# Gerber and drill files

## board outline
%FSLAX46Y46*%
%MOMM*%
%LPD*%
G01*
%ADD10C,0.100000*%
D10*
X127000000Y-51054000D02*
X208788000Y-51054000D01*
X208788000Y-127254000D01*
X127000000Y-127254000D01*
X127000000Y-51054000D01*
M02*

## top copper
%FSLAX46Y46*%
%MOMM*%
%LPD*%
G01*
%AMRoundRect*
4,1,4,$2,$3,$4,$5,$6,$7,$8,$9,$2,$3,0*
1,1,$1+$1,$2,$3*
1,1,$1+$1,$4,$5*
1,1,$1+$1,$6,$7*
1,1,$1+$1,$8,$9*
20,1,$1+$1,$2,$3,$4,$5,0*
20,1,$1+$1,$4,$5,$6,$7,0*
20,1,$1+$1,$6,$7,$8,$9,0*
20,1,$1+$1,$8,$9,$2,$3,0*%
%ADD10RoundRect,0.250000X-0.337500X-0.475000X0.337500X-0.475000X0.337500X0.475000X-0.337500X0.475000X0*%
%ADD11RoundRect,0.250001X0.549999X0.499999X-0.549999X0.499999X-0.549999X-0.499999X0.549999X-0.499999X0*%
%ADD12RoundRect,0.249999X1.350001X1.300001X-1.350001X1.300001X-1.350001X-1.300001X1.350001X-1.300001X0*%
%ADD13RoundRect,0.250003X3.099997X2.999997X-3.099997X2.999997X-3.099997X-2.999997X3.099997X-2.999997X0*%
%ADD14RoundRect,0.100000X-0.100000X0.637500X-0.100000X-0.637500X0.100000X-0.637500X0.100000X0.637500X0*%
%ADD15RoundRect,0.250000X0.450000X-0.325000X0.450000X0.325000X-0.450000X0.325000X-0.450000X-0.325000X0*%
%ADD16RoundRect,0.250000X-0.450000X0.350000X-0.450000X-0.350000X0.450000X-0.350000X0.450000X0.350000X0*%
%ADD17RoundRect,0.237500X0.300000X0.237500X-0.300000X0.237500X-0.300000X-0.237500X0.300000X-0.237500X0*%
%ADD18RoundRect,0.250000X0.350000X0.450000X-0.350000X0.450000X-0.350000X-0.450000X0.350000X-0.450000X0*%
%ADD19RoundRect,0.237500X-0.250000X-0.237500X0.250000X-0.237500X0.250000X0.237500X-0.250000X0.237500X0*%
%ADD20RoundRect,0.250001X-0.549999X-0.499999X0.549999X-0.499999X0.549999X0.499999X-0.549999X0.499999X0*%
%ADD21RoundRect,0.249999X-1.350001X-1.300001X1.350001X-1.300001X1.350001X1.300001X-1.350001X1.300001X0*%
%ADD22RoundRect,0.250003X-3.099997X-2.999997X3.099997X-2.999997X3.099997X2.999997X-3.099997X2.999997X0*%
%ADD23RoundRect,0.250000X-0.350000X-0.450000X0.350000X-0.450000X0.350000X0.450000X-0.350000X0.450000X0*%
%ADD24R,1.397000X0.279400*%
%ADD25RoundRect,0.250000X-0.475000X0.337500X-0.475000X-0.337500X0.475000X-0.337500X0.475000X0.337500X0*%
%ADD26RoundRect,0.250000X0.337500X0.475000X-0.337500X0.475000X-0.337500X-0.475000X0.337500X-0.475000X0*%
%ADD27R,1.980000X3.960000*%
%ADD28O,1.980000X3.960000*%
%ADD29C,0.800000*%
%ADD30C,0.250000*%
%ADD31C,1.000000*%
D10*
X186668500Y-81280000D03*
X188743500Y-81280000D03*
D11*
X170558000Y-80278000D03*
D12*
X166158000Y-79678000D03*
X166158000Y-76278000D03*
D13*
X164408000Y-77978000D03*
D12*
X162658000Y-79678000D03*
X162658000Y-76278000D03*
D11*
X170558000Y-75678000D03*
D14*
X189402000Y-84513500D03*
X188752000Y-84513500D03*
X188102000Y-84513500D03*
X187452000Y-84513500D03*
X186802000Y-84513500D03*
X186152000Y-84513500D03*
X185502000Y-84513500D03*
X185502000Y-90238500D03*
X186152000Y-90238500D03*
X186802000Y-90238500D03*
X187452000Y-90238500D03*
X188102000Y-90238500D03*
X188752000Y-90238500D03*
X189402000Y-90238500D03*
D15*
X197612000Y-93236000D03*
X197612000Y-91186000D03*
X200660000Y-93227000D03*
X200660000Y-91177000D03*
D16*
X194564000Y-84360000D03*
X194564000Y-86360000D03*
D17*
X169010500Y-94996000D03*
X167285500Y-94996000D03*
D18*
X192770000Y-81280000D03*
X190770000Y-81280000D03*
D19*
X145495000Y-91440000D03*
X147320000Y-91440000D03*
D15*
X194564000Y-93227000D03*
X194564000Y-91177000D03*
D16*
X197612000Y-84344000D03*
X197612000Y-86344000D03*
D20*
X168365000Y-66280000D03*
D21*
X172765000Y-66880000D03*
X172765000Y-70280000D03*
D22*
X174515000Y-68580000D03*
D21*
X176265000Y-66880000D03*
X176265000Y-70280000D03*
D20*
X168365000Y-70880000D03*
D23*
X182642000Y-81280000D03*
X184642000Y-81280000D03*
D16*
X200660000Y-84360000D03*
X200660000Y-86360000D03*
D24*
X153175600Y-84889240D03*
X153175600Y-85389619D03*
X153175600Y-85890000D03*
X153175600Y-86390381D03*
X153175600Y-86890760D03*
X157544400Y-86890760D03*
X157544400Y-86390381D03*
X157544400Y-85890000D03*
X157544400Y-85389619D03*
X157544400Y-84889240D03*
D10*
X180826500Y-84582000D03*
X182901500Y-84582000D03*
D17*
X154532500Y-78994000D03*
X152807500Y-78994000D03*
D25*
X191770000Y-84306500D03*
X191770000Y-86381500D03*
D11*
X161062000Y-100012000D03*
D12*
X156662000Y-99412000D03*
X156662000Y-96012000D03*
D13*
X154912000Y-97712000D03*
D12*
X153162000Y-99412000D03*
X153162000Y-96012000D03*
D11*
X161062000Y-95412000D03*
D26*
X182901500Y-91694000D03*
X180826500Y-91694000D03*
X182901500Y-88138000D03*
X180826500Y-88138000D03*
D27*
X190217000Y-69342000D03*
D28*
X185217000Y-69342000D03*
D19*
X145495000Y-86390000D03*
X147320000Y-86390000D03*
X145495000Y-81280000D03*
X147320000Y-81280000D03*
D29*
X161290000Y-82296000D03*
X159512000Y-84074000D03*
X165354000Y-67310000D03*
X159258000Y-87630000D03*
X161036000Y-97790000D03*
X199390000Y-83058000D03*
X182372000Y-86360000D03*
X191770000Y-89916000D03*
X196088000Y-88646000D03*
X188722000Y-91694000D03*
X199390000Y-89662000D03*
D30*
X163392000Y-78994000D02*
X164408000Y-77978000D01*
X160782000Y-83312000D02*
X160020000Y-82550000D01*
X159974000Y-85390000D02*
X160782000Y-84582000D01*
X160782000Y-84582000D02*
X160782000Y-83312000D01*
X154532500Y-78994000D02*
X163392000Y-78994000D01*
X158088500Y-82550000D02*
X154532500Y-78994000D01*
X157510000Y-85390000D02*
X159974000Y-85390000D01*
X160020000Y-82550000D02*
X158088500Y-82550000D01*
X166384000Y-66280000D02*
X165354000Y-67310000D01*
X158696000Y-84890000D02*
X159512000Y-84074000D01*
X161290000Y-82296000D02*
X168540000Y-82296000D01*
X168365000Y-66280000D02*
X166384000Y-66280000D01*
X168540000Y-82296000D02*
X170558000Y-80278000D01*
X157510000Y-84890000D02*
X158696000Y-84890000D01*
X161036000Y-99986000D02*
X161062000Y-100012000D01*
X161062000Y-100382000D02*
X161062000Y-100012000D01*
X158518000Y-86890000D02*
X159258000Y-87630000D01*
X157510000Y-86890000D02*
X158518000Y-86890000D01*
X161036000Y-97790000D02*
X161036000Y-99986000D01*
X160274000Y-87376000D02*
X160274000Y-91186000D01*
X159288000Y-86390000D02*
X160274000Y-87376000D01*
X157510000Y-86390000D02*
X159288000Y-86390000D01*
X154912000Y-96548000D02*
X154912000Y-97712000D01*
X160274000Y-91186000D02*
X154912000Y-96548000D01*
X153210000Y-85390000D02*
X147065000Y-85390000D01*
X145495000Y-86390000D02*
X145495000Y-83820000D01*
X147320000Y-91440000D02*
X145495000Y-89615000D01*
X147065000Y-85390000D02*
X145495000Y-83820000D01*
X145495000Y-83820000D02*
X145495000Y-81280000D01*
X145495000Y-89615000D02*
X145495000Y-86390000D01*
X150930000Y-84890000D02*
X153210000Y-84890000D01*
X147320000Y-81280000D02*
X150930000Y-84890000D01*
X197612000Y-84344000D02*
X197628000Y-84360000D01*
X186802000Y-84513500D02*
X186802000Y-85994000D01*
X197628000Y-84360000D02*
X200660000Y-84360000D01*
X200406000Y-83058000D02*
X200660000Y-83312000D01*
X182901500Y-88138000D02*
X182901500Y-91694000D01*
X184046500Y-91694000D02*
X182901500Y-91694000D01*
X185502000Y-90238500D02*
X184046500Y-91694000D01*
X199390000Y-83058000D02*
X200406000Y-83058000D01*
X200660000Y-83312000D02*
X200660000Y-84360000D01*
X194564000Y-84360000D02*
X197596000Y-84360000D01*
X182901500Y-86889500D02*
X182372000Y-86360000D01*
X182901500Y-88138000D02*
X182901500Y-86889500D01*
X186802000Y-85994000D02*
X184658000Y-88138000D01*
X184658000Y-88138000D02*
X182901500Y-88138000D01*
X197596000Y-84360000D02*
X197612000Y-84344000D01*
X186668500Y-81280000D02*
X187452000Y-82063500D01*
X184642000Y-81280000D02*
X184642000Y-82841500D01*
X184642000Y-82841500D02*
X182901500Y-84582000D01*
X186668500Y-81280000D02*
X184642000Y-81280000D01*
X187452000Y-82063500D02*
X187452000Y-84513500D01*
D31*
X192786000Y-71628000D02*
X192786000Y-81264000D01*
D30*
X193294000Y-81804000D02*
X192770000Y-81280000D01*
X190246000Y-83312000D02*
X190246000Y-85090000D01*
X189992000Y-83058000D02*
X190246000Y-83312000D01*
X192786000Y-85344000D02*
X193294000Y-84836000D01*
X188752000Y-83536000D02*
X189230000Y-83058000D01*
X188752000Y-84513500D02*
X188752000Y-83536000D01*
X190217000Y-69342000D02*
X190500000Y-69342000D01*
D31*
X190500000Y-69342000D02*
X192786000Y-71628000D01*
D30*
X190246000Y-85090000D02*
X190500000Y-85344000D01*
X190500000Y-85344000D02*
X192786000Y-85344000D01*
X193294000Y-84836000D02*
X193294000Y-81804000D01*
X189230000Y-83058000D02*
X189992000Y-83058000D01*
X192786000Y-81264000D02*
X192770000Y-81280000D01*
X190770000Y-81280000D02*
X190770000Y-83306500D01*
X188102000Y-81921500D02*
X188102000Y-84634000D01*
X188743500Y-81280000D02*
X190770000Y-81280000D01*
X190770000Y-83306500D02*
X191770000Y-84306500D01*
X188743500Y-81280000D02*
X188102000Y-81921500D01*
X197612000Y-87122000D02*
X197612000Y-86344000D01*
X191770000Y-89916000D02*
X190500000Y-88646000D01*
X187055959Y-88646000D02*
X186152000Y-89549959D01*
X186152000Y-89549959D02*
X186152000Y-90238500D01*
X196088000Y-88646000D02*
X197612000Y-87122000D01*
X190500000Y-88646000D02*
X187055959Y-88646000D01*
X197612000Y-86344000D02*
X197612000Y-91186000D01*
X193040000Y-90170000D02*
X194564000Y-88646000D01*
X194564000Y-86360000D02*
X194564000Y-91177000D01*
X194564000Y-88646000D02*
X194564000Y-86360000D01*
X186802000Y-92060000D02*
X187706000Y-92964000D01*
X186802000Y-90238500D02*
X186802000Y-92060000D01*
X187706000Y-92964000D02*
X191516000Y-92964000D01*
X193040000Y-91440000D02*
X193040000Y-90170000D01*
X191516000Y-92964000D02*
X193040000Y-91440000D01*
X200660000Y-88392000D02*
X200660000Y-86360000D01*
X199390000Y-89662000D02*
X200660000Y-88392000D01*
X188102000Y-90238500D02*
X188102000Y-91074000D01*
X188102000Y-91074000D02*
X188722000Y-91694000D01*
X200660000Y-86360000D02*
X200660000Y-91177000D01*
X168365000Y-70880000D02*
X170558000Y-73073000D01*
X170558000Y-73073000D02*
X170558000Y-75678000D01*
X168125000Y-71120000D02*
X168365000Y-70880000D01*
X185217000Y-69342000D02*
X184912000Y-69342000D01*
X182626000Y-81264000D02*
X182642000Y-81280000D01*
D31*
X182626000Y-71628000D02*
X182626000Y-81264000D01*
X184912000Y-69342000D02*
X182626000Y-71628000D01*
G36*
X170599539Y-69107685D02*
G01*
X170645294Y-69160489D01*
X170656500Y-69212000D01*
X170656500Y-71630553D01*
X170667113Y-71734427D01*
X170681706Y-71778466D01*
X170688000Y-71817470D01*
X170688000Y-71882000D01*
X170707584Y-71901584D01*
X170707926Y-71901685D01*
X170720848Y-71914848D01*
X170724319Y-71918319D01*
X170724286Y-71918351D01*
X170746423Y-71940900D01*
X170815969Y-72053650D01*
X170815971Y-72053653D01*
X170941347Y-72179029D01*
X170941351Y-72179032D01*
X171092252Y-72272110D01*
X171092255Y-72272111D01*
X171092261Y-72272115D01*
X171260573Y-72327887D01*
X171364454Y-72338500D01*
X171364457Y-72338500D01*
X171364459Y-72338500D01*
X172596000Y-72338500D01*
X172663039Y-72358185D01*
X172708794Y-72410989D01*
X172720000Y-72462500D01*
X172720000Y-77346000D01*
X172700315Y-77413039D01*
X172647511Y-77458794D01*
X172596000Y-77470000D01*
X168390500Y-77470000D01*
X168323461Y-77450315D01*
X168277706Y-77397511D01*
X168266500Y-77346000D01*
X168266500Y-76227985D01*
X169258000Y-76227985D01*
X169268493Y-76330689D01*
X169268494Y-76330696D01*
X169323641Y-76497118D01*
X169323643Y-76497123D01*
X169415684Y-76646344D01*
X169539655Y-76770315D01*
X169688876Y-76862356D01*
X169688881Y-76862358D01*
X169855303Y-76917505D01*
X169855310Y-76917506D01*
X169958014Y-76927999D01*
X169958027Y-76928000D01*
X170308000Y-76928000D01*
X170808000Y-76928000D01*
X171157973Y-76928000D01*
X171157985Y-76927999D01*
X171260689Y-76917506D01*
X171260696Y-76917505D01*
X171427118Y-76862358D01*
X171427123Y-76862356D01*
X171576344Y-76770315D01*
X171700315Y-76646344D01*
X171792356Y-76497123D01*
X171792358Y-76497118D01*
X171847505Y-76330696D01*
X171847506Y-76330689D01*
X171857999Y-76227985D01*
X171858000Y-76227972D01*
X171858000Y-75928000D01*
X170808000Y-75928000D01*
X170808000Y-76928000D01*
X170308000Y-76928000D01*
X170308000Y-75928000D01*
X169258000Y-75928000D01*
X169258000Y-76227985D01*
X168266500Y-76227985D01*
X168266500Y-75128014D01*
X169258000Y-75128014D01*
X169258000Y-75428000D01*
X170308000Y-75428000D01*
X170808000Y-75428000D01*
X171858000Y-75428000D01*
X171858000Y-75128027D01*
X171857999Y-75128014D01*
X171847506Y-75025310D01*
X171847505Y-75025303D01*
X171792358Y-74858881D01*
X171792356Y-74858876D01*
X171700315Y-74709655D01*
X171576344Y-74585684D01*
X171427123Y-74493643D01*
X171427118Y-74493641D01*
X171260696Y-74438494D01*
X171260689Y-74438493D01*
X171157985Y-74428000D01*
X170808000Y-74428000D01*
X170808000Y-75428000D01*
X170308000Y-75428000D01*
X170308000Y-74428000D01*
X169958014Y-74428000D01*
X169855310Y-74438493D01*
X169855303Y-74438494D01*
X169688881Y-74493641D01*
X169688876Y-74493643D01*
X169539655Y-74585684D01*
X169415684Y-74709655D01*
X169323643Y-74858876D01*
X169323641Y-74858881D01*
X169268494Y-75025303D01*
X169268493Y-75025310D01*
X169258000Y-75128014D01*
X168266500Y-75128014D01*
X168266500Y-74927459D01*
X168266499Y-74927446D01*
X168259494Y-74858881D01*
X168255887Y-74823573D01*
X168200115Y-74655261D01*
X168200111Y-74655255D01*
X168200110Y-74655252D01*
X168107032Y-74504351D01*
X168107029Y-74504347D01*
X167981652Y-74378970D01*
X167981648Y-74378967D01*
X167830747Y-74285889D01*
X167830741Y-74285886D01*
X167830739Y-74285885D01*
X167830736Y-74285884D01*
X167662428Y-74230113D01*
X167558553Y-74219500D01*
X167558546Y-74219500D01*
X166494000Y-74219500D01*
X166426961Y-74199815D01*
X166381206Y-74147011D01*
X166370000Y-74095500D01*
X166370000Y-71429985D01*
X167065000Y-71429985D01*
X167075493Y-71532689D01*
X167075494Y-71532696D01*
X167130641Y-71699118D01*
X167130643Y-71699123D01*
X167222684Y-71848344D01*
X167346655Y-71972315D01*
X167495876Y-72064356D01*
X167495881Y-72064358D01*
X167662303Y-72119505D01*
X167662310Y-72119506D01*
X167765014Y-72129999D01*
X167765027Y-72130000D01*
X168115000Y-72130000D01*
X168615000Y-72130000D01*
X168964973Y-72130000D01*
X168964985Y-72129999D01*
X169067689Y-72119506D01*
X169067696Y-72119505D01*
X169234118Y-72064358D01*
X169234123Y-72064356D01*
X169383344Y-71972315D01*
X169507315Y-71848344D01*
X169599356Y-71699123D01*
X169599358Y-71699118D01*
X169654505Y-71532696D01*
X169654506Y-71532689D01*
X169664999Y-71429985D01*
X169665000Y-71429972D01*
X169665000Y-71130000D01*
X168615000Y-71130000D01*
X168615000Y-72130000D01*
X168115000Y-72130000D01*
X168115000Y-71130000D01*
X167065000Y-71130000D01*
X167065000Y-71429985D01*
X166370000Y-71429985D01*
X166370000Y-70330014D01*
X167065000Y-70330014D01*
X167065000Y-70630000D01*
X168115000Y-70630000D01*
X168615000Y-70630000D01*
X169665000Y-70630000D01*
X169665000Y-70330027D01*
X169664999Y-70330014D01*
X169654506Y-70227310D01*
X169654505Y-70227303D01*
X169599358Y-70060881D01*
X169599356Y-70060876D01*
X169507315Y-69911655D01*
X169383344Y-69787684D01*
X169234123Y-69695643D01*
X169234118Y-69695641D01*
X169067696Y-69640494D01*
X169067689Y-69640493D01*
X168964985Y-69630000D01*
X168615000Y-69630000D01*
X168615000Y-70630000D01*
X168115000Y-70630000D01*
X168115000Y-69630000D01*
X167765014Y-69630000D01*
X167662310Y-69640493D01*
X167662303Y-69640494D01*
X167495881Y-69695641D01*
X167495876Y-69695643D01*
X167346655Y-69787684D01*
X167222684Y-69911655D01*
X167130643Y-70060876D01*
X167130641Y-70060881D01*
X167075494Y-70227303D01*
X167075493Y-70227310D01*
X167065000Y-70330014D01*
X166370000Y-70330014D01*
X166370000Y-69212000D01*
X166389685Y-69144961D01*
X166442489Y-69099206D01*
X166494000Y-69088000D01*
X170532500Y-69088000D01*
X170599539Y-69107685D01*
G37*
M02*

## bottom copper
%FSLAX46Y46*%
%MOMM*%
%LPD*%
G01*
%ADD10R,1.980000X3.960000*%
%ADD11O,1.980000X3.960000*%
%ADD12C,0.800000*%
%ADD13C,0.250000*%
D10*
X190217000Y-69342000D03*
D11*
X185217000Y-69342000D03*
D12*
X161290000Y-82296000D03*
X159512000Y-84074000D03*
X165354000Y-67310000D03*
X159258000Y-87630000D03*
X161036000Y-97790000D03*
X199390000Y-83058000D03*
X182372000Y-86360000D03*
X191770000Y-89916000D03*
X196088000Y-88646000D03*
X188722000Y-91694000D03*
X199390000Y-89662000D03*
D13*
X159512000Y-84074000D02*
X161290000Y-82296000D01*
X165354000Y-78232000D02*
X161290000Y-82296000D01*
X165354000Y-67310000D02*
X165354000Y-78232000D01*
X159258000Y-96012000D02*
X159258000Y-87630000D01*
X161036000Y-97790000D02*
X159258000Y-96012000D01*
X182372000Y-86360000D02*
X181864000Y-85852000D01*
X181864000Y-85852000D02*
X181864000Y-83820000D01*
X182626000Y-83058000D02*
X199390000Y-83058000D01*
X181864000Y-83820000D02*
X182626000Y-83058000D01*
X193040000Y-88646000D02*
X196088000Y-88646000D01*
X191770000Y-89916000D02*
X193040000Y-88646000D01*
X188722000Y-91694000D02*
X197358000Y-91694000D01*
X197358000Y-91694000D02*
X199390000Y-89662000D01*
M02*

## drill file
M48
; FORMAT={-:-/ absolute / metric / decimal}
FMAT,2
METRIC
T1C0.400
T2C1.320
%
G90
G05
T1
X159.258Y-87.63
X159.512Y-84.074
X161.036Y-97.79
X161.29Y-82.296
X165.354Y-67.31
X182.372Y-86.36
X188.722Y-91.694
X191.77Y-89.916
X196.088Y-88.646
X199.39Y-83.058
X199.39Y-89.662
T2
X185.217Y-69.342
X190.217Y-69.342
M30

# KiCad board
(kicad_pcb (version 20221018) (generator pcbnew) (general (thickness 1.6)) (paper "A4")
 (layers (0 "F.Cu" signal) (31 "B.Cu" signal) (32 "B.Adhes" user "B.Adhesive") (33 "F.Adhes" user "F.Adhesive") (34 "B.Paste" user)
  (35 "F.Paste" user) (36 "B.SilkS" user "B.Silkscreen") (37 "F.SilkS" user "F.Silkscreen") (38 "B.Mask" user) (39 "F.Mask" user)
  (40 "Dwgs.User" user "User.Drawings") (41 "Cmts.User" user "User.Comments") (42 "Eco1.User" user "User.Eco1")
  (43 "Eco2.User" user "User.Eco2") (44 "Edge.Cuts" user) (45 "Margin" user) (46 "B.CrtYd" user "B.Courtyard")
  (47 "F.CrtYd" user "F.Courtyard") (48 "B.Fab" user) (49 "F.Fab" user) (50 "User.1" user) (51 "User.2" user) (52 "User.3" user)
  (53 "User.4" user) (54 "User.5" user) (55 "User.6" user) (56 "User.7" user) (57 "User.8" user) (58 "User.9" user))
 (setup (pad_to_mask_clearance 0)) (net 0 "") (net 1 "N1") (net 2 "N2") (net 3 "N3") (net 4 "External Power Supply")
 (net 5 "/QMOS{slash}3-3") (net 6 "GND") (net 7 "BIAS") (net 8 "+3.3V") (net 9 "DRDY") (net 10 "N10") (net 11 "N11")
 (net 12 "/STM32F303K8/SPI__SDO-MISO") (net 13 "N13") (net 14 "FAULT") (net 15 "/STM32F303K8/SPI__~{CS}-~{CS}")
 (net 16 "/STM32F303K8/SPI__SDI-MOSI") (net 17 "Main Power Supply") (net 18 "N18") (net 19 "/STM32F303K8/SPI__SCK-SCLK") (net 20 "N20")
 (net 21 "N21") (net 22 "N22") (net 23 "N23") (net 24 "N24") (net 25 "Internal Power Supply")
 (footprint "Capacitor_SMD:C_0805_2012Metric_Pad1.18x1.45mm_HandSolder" (layer "F.Cu") (at 187.706 81.28)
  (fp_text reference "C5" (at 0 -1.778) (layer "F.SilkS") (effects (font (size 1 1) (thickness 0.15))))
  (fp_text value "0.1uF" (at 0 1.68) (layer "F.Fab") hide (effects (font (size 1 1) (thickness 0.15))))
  (pad "1" smd roundrect (at -1.0375 0) (size 1.175 1.45) (layers "F.Cu" "F.Paste" "F.Mask") (roundrect_rratio 0.212766) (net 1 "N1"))
  (pad "2" smd roundrect (at 1.0375 0) (size 1.175 1.45) (layers "F.Cu" "F.Paste" "F.Mask") (roundrect_rratio 0.212766) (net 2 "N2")))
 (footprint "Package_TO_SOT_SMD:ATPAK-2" (layer "F.Cu") (at 165.608 77.978 180)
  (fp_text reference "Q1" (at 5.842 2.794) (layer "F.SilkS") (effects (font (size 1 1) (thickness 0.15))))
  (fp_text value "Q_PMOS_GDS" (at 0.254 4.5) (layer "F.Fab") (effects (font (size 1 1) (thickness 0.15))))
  (pad "1" smd roundrect (at -4.95 -2.3 180) (size 1.6 1.5) (layers "F.Cu" "F.Paste" "F.Mask") (roundrect_rratio 0.166667) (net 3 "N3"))
  (pad "2" smd roundrect (at -0.55 -1.7 180) (size 3.2 3.1) (layers "F.Cu" "F.Paste") (roundrect_rratio 0.080645)
   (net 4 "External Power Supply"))
  (pad "2" smd roundrect (at -0.55 1.7 180) (size 3.2 3.1) (layers "F.Cu" "F.Paste") (roundrect_rratio 0.080645)
   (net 4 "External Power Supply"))
  (pad "2" smd roundrect (at 1.2 0 180) (size 6.7 6.5) (layers "F.Cu" "F.Mask") (roundrect_rratio 0.038462) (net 4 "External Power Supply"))
  (pad "2" smd roundrect (at 2.95 -1.7 180) (size 3.2 3.1) (layers "F.Cu" "F.Paste") (roundrect_rratio 0.080645)
   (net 4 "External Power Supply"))
  (pad "2" smd roundrect (at 2.95 1.7 180) (size 3.2 3.1) (layers "F.Cu" "F.Paste") (roundrect_rratio 0.080645)
   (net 4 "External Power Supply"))
  (pad "3" smd roundrect (at -4.95 2.3 180) (size 1.6 1.5) (layers "F.Cu" "F.Paste" "F.Mask") (roundrect_rratio 0.166667)
   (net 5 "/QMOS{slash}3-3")))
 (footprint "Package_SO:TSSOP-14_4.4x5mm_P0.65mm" (layer "F.Cu") (at 187.452 87.376 -90)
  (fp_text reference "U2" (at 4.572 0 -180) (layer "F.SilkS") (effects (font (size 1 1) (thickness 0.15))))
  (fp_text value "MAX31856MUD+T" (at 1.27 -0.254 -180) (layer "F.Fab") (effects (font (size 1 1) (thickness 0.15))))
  (pad "1" smd roundrect (at -2.8625 -1.95 270) (size 1.475 0.4) (layers "F.Cu" "F.Paste" "F.Mask") (roundrect_rratio 0.25) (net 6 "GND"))
  (pad "2" smd roundrect (at -2.8625 -1.3 270) (size 1.475 0.4) (layers "F.Cu" "F.Paste" "F.Mask") (roundrect_rratio 0.25) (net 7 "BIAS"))
  (pad "3" smd roundrect (at -2.8625 -0.65 270) (size 1.475 0.4) (layers "F.Cu" "F.Paste" "F.Mask") (roundrect_rratio 0.25) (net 2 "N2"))
  (pad "4" smd roundrect (at -2.8625 0 270) (size 1.475 0.4) (layers "F.Cu" "F.Paste" "F.Mask") (roundrect_rratio 0.25) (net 1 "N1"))
  (pad "5" smd roundrect (at -2.8625 0.65 270) (size 1.475 0.4) (layers "F.Cu" "F.Paste" "F.Mask") (roundrect_rratio 0.25) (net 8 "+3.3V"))
  (pad "6" smd roundrect (at -2.8625 1.3 270) (size 1.475 0.4) (layers "F.Cu" "F.Paste" "F.Mask") (roundrect_rratio 0.25))
  (pad "7" smd roundrect (at -2.8625 1.95 270) (size 1.475 0.4) (layers "F.Cu" "F.Paste" "F.Mask") (roundrect_rratio 0.25) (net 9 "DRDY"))
  (pad "8" smd roundrect (at 2.8625 1.95 270) (size 1.475 0.4) (layers "F.Cu" "F.Paste" "F.Mask") (roundrect_rratio 0.25) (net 8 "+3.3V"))
  (pad "9" smd roundrect (at 2.8625 1.3 270) (size 1.475 0.4) (layers "F.Cu" "F.Paste" "F.Mask") (roundrect_rratio 0.25) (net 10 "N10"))
  (pad "10" smd roundrect (at 2.8625 0.65 270) (size 1.475 0.4) (layers "F.Cu" "F.Paste" "F.Mask") (roundrect_rratio 0.25) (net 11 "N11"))
  (pad "11" smd roundrect (at 2.8625 0 270) (size 1.475 0.4) (layers "F.Cu" "F.Paste" "F.Mask") (roundrect_rratio 0.25)
   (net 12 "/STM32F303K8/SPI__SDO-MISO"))
  (pad "12" smd roundrect (at 2.8625 -0.65 270) (size 1.475 0.4) (layers "F.Cu" "F.Paste" "F.Mask") (roundrect_rratio 0.25) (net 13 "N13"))
  (pad "13" smd roundrect (at 2.8625 -1.3 270) (size 1.475 0.4) (layers "F.Cu" "F.Paste" "F.Mask") (roundrect_rratio 0.25) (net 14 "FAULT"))
  (pad "14" smd roundrect (at 2.8625 -1.95 270) (size 1.475 0.4) (layers "F.Cu" "F.Paste" "F.Mask") (roundrect_rratio 0.25) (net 6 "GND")))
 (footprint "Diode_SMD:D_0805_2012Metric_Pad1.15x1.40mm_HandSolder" (layer "F.Cu") (at 197.612 92.211 90)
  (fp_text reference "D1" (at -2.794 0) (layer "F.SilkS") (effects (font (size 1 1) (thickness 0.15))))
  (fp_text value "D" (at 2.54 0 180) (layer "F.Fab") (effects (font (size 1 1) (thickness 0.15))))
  (pad "1" smd roundrect (at -1.025 0 90) (size 1.15 1.4) (layers "F.Cu" "F.Paste" "F.Mask") (roundrect_rratio 0.217391)
   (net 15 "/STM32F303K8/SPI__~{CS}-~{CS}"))
  (pad "2" smd roundrect (at 1.025 0 90) (size 1.15 1.4) (layers "F.Cu" "F.Paste" "F.Mask") (roundrect_rratio 0.217391) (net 10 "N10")))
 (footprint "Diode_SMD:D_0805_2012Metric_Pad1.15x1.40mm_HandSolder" (layer "F.Cu") (at 200.66 92.202 90)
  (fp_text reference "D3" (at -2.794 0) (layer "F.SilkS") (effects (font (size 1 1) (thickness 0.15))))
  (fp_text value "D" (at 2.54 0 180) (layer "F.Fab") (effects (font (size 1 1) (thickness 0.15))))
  (pad "1" smd roundrect (at -1.025 0 90) (size 1.15 1.4) (layers "F.Cu" "F.Paste" "F.Mask") (roundrect_rratio 0.217391)
   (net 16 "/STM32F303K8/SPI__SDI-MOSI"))
  (pad "2" smd roundrect (at 1.025 0 90) (size 1.15 1.4) (layers "F.Cu" "F.Paste" "F.Mask") (roundrect_rratio 0.217391) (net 13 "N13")))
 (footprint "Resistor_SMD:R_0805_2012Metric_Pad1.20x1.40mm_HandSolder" (layer "F.Cu") (at 194.564 85.36 -90)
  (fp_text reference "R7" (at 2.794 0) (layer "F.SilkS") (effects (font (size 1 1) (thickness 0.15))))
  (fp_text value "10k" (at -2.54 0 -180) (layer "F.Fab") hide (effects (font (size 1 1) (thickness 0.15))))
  (pad "1" smd roundrect (at -1 0 270) (size 1.2 1.4) (layers "F.Cu" "F.Paste" "F.Mask") (roundrect_rratio 0.208333) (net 8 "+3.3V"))
  (pad "2" smd roundrect (at 1 0 270) (size 1.2 1.4) (layers "F.Cu" "F.Paste" "F.Mask") (roundrect_rratio 0.208333) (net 11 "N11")))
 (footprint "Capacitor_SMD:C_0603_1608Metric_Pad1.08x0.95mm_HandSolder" (layer "F.Cu") (at 168.148 94.996 180)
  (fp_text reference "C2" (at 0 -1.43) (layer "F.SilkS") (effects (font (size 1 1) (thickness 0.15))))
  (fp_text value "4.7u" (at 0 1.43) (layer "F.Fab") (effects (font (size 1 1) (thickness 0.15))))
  (pad "1" smd roundrect (at -0.8625 0 180) (size 1.075 0.95) (layers "F.Cu" "F.Paste" "F.Mask") (roundrect_rratio 0.25)
   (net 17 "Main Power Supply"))
  (pad "2" smd roundrect (at 0.8625 0 180) (size 1.075 0.95) (layers "F.Cu" "F.Paste" "F.Mask") (roundrect_rratio 0.25) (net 6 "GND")))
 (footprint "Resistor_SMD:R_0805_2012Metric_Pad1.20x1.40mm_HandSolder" (layer "F.Cu") (at 191.77 81.28 180)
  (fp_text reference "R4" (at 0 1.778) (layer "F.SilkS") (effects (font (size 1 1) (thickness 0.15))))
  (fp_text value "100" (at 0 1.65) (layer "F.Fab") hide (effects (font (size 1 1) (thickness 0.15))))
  (pad "1" smd roundrect (at -1 0 180) (size 1.2 1.4) (layers "F.Cu" "F.Paste" "F.Mask") (roundrect_rratio 0.208333) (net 7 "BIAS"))
  (pad "2" smd roundrect (at 1 0 180) (size 1.2 1.4) (layers "F.Cu" "F.Paste" "F.Mask") (roundrect_rratio 0.208333) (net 2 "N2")))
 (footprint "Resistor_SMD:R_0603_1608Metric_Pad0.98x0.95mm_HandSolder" (layer "F.Cu") (at 146.4075 91.44)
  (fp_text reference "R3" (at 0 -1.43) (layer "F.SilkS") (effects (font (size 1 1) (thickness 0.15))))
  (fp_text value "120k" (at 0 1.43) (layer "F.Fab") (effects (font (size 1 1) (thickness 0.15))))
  (pad "1" smd roundrect (at -0.9125 0) (size 0.975 0.95) (layers "F.Cu" "F.Paste" "F.Mask") (roundrect_rratio 0.25)
   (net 4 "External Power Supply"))
  (pad "2" smd roundrect (at 0.9125 0) (size 0.975 0.95) (layers "F.Cu" "F.Paste" "F.Mask") (roundrect_rratio 0.25) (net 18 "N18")))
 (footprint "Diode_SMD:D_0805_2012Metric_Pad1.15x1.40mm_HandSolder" (layer "F.Cu") (at 194.564 92.202 90)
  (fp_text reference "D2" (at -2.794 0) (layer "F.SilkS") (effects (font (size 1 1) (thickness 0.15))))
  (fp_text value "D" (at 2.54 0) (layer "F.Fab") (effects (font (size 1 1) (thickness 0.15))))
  (pad "1" smd roundrect (at -1.025 0 90) (size 1.15 1.4) (layers "F.Cu" "F.Paste" "F.Mask") (roundrect_rratio 0.217391)
   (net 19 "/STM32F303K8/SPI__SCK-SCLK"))
  (pad "2" smd roundrect (at 1.025 0 90) (size 1.15 1.4) (layers "F.Cu" "F.Paste" "F.Mask") (roundrect_rratio 0.217391) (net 11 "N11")))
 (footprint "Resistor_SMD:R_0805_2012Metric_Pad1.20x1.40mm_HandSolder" (layer "F.Cu") (at 197.612 85.344 -90)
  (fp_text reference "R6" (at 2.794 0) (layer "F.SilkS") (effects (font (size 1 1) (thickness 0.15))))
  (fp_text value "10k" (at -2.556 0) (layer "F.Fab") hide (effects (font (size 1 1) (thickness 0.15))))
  (pad "1" smd roundrect (at -1 0 270) (size 1.2 1.4) (layers "F.Cu" "F.Paste" "F.Mask") (roundrect_rratio 0.208333) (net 8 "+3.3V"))
  (pad "2" smd roundrect (at 1 0 270) (size 1.2 1.4) (layers "F.Cu" "F.Paste" "F.Mask") (roundrect_rratio 0.208333) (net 10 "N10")))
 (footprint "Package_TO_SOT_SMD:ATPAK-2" (layer "F.Cu") (at 173.315 68.58)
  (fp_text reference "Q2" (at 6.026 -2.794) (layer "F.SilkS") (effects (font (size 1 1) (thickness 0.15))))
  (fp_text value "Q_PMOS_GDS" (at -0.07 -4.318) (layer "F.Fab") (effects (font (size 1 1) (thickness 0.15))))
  (pad "1" smd roundrect (at -4.95 -2.3) (size 1.6 1.5) (layers "F.Cu" "F.Paste" "F.Mask") (roundrect_rratio 0.166667) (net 3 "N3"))
  (pad "2" smd roundrect (at -0.55 -1.7) (size 3.2 3.1) (layers "F.Cu" "F.Paste") (roundrect_rratio 0.080645) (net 17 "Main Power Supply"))
  (pad "2" smd roundrect (at -0.55 1.7) (size 3.2 3.1) (layers "F.Cu" "F.Paste") (roundrect_rratio 0.080645) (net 17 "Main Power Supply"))
  (pad "2" smd roundrect (at 1.2 0) (size 6.7 6.5) (layers "F.Cu" "F.Mask") (roundrect_rratio 0.038462) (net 17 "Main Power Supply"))
  (pad "2" smd roundrect (at 2.95 -1.7) (size 3.2 3.1) (layers "F.Cu" "F.Paste") (roundrect_rratio 0.080645) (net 17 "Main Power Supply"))
  (pad "2" smd roundrect (at 2.95 1.7) (size 3.2 3.1) (layers "F.Cu" "F.Paste") (roundrect_rratio 0.080645) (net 17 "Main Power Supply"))
  (pad "3" smd roundrect (at -4.95 2.3) (size 1.6 1.5) (layers "F.Cu" "F.Paste" "F.Mask") (roundrect_rratio 0.166667)
   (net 5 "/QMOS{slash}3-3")))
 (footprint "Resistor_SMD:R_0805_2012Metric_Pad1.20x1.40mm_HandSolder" (layer "F.Cu") (at 183.642 81.28)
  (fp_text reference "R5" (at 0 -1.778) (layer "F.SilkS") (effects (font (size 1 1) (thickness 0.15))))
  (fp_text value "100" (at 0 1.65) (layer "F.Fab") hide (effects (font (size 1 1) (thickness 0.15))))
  (pad "1" smd roundrect (at -1 0) (size 1.2 1.4) (layers "F.Cu" "F.Paste" "F.Mask") (roundrect_rratio 0.208333) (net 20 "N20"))
  (pad "2" smd roundrect (at 1 0) (size 1.2 1.4) (layers "F.Cu" "F.Paste" "F.Mask") (roundrect_rratio 0.208333) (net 1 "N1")))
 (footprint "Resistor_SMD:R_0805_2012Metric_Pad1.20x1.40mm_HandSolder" (layer "F.Cu") (at 200.66 85.36 -90)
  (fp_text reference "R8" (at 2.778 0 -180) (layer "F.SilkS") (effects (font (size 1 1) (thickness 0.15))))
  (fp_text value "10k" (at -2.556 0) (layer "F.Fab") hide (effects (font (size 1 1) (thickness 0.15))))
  (pad "1" smd roundrect (at -1 0 270) (size 1.2 1.4) (layers "F.Cu" "F.Paste" "F.Mask") (roundrect_rratio 0.208333) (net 8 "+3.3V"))
  (pad "2" smd roundrect (at 1 0 270) (size 1.2 1.4) (layers "F.Cu" "F.Paste" "F.Mask") (roundrect_rratio 0.208333) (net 13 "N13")))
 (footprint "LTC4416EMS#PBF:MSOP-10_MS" (layer "F.Cu") (at 155.36 85.89)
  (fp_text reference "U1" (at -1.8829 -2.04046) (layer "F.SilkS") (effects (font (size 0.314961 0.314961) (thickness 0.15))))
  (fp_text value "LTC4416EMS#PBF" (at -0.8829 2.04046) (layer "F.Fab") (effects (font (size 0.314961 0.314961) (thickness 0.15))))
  (pad "1" smd rect (at -2.1844 -1.00076) (size 1.397 0.2794) (layers "F.Cu" "F.Paste" "F.Mask") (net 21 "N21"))
  (pad "2" smd rect (at -2.1844 -0.500381) (size 1.397 0.2794) (layers "F.Cu" "F.Paste" "F.Mask") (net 18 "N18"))
  (pad "3" smd rect (at -2.1844 0) (size 1.397 0.2794) (layers "F.Cu" "F.Paste" "F.Mask") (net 6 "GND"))
  (pad "4" smd rect (at -2.1844 0.500381) (size 1.397 0.2794) (layers "F.Cu" "F.Paste" "F.Mask") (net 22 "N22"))
  (pad "5" smd rect (at -2.1844 1.00076) (size 1.397 0.2794) (layers "F.Cu" "F.Paste" "F.Mask") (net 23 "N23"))
  (pad "6" smd rect (at 2.1844 1.00076) (size 1.397 0.2794) (layers "F.Cu" "F.Paste" "F.Mask") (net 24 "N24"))
  (pad "7" smd rect (at 2.1844 0.500381) (size 1.397 0.2794) (layers "F.Cu" "F.Paste" "F.Mask") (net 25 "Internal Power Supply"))
  (pad "8" smd rect (at 2.1844 0) (size 1.397 0.2794) (layers "F.Cu" "F.Paste" "F.Mask") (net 17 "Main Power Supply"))
  (pad "9" smd rect (at 2.1844 -0.500381) (size 1.397 0.2794) (layers "F.Cu" "F.Paste" "F.Mask") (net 4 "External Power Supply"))
  (pad "10" smd rect (at 2.1844 -1.00076) (size 1.397 0.2794) (layers "F.Cu" "F.Paste" "F.Mask") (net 3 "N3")))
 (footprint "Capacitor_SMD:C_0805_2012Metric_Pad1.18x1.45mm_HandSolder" (layer "F.Cu") (at 181.864 84.582)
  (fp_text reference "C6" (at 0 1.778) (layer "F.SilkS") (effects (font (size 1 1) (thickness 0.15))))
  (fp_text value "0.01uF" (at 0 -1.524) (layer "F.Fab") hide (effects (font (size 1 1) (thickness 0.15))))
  (pad "1" smd roundrect (at -1.0375 0) (size 1.175 1.45) (layers "F.Cu" "F.Paste" "F.Mask") (roundrect_rratio 0.212766) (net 6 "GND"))
  (pad "2" smd roundrect (at 1.0375 0) (size 1.175 1.45) (layers "F.Cu" "F.Paste" "F.Mask") (roundrect_rratio 0.212766) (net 1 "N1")))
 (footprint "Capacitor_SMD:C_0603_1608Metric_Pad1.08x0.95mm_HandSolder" (layer "F.Cu") (at 153.67 78.994 180)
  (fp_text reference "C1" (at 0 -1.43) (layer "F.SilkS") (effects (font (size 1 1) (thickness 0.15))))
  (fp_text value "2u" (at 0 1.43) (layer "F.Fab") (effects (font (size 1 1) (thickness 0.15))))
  (pad "1" smd roundrect (at -0.8625 0 180) (size 1.075 0.95) (layers "F.Cu" "F.Paste" "F.Mask") (roundrect_rratio 0.25)
   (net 4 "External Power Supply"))
  (pad "2" smd roundrect (at 0.8625 0 180) (size 1.075 0.95) (layers "F.Cu" "F.Paste" "F.Mask") (roundrect_rratio 0.25) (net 6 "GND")))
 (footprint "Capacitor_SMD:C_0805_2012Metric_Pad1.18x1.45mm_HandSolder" (layer "F.Cu") (at 191.77 85.344 -90)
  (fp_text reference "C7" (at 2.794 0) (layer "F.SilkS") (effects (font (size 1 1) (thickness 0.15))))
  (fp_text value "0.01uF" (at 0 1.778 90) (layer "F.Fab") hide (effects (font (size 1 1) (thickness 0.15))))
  (pad "1" smd roundrect (at -1.0375 0 270) (size 1.175 1.45) (layers "F.Cu" "F.Paste" "F.Mask") (roundrect_rratio 0.212766) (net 2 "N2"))
  (pad "2" smd roundrect (at 1.0375 0 270) (size 1.175 1.45) (layers "F.Cu" "F.Paste" "F.Mask") (roundrect_rratio 0.212766) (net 6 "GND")))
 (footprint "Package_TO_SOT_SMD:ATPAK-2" (layer "F.Cu") (at 156.112 97.712 180)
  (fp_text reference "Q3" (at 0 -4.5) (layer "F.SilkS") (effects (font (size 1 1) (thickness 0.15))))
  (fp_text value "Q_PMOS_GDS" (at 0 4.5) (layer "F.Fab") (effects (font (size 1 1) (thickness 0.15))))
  (pad "1" smd roundrect (at -4.95 -2.3 180) (size 1.6 1.5) (layers "F.Cu" "F.Paste" "F.Mask") (roundrect_rratio 0.166667) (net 24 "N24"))
  (pad "2" smd roundrect (at -0.55 -1.7 180) (size 3.2 3.1) (layers "F.Cu" "F.Paste") (roundrect_rratio 0.080645)
   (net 25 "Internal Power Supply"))
  (pad "2" smd roundrect (at -0.55 1.7 180) (size 3.2 3.1) (layers "F.Cu" "F.Paste") (roundrect_rratio 0.080645)
   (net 25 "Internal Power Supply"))
  (pad "2" smd roundrect (at 1.2 0 180) (size 6.7 6.5) (layers "F.Cu" "F.Mask") (roundrect_rratio 0.038462) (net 25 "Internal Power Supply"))
  (pad "2" smd roundrect (at 2.95 -1.7 180) (size 3.2 3.1) (layers "F.Cu" "F.Paste") (roundrect_rratio 0.080645)
   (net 25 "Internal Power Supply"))
  (pad "2" smd roundrect (at 2.95 1.7 180) (size 3.2 3.1) (layers "F.Cu" "F.Paste") (roundrect_rratio 0.080645)
   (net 25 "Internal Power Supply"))
  (pad "3" smd roundrect (at -4.95 2.3 180) (size 1.6 1.5) (layers "F.Cu" "F.Paste" "F.Mask") (roundrect_rratio 0.166667)
   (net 17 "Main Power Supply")))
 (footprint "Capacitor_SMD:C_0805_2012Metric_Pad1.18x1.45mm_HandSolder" (layer "F.Cu") (at 181.864 91.694 180)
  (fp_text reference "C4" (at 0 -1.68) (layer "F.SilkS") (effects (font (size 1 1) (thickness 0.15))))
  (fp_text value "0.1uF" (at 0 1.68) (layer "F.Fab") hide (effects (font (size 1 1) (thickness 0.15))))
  (pad "1" smd roundrect (at -1.0375 0 180) (size 1.175 1.45) (layers "F.Cu" "F.Paste" "F.Mask") (roundrect_rratio 0.212766) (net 8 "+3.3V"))
  (pad "2" smd roundrect (at 1.0375 0 180) (size 1.175 1.45) (layers "F.Cu" "F.Paste" "F.Mask") (roundrect_rratio 0.212766) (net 6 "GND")))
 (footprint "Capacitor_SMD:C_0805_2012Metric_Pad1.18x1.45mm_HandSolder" (layer "F.Cu") (at 181.864 88.138 180)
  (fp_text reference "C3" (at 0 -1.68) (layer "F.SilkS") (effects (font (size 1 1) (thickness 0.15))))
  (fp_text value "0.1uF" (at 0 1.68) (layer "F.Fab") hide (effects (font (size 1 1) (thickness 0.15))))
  (pad "1" smd roundrect (at -1.0375 0 180) (size 1.175 1.45) (layers "F.Cu" "F.Paste" "F.Mask") (roundrect_rratio 0.212766) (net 8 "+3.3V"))
  (pad "2" smd roundrect (at 1.0375 0 180) (size 1.175 1.45) (layers "F.Cu" "F.Paste" "F.Mask") (roundrect_rratio 0.212766) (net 6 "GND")))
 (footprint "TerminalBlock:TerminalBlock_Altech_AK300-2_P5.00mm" (layer "F.Cu") (at 190.217 69.342 180)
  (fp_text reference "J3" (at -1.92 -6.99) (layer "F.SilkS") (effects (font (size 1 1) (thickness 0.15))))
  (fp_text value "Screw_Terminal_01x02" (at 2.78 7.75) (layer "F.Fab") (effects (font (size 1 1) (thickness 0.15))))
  (pad "1" thru_hole rect (at 0 0 180) (size 1.98 3.96) (drill 1.32) (layers "*.Cu" "*.Mask") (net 7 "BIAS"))
  (pad "2" thru_hole oval (at 5 0 180) (size 1.98 3.96) (drill 1.32) (layers "*.Cu" "*.Mask") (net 20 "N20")))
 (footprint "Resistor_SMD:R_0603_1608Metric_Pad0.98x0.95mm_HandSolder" (layer "F.Cu") (at 146.4075 86.39)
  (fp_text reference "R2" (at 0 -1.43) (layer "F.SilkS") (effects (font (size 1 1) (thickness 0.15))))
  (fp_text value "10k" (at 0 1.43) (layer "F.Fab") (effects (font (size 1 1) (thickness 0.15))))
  (pad "1" smd roundrect (at -0.9125 0) (size 0.975 0.95) (layers "F.Cu" "F.Paste" "F.Mask") (roundrect_rratio 0.25) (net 18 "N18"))
  (pad "2" smd roundrect (at 0.9125 0) (size 0.975 0.95) (layers "F.Cu" "F.Paste" "F.Mask") (roundrect_rratio 0.25) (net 6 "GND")))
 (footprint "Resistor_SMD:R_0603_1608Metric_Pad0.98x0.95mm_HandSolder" (layer "F.Cu") (at 146.4075 81.28)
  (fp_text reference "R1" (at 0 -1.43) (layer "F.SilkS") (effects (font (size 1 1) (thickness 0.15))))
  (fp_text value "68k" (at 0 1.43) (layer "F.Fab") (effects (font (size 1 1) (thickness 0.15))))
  (pad "1" smd roundrect (at -0.9125 0) (size 0.975 0.95) (layers "F.Cu" "F.Paste" "F.Mask") (roundrect_rratio 0.25) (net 18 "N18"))
  (pad "2" smd roundrect (at 0.9125 0) (size 0.975 0.95) (layers "F.Cu" "F.Paste" "F.Mask") (roundrect_rratio 0.25) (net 21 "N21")))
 (gr_rect (start 127 51.054) (end 208.788 127.254) (stroke (width 0.1) (type default)) (fill none) (layer "Edge.Cuts"))
 (segment (start 163.392 78.994) (end 164.408 77.978) (width 0.25) (layer "F.Cu") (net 4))
 (segment (start 160.782 83.312) (end 160.02 82.55) (width 0.25) (layer "F.Cu") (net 4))
 (segment (start 159.974 85.39) (end 160.782 84.582) (width 0.25) (layer "F.Cu") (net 4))
 (segment (start 160.782 84.582) (end 160.782 83.312) (width 0.25) (layer "F.Cu") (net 4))
 (segment (start 154.5325 78.994) (end 163.392 78.994) (width 0.25) (layer "F.Cu") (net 4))
 (segment (start 158.0885 82.55) (end 154.5325 78.994) (width 0.25) (layer "F.Cu") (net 4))
 (segment (start 157.51 85.39) (end 159.974 85.39) (width 0.25) (layer "F.Cu") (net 4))
 (segment (start 160.02 82.55) (end 158.0885 82.55) (width 0.25) (layer "F.Cu") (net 4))
 (segment (start 166.384 66.28) (end 165.354 67.31) (width 0.25) (layer "F.Cu") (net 3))
 (segment (start 158.696 84.89) (end 159.512 84.074) (width 0.25) (layer "F.Cu") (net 3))
 (segment (start 161.29 82.296) (end 168.54 82.296) (width 0.25) (layer "F.Cu") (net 3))
 (segment (start 168.365 66.28) (end 166.384 66.28) (width 0.25) (layer "F.Cu") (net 3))
 (segment (start 168.54 82.296) (end 170.558 80.278) (width 0.25) (layer "F.Cu") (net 3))
 (segment (start 157.51 84.89) (end 158.696 84.89) (width 0.25) (layer "F.Cu") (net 3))
 (via (at 161.29 82.296) (size 0.8) (drill 0.4) (layers "F.Cu" "B.Cu") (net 3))
 (via (at 159.512 84.074) (size 0.8) (drill 0.4) (layers "F.Cu" "B.Cu") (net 3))
 (via (at 165.354 67.31) (size 0.8) (drill 0.4) (layers "F.Cu" "B.Cu") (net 3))
 (segment (start 159.512 84.074) (end 161.29 82.296) (width 0.25) (layer "B.Cu") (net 3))
 (segment (start 165.354 78.232) (end 161.29 82.296) (width 0.25) (layer "B.Cu") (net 3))
 (segment (start 165.354 67.31) (end 165.354 78.232) (width 0.25) (layer "B.Cu") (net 3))
 (segment (start 161.036 99.986) (end 161.062 100.012) (width 0.25) (layer "F.Cu") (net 24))
 (segment (start 161.062 100.382) (end 161.062 100.012) (width 0.25) (layer "F.Cu") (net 24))
 (segment (start 158.518 86.89) (end 159.258 87.63) (width 0.25) (layer "F.Cu") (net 24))
 (segment (start 157.51 86.89) (end 158.518 86.89) (width 0.25) (layer "F.Cu") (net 24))
 (segment (start 161.036 97.79) (end 161.036 99.986) (width 0.25) (layer "F.Cu") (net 24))
 (via (at 159.258 87.63) (size 0.8) (drill 0.4) (layers "F.Cu" "B.Cu") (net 24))
 (via (at 161.036 97.79) (size 0.8) (drill 0.4) (layers "F.Cu" "B.Cu") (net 24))
 (segment (start 159.258 96.012) (end 159.258 87.63) (width 0.25) (layer "B.Cu") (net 24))
 (segment (start 161.036 97.79) (end 159.258 96.012) (width 0.25) (layer "B.Cu") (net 24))
 (segment (start 160.274 87.376) (end 160.274 91.186) (width 0.25) (layer "F.Cu") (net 25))
 (segment (start 159.288 86.39) (end 160.274 87.376) (width 0.25) (layer "F.Cu") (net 25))
 (segment (start 157.51 86.39) (end 159.288 86.39) (width 0.25) (layer "F.Cu") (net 25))
 (segment (start 154.912 96.548) (end 154.912 97.712) (width 0.25) (layer "F.Cu") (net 25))
 (segment (start 160.274 91.186) (end 154.912 96.548) (width 0.25) (layer "F.Cu") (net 25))
 (segment (start 153.21 85.39) (end 147.065 85.39) (width 0.25) (layer "F.Cu") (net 18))
 (segment (start 145.495 86.39) (end 145.495 83.82) (width 0.25) (layer "F.Cu") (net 18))
 (segment (start 147.32 91.44) (end 145.495 89.615) (width 0.25) (layer "F.Cu") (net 18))
 (segment (start 147.065 85.39) (end 145.495 83.82) (width 0.25) (layer "F.Cu") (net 18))
 (segment (start 145.495 83.82) (end 145.495 81.28) (width 0.25) (layer "F.Cu") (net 18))
 (segment (start 145.495 89.615) (end 145.495 86.39) (width 0.25) (layer "F.Cu") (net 18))
 (segment (start 150.93 84.89) (end 153.21 84.89) (width 0.25) (layer "F.Cu") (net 21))
 (segment (start 147.32 81.28) (end 150.93 84.89) (width 0.25) (layer "F.Cu") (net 21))
 (segment (start 197.612 84.344) (end 197.628 84.36) (width 0.25) (layer "F.Cu") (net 8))
 (segment (start 186.802 84.5135) (end 186.802 85.994) (width 0.25) (layer "F.Cu") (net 8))
 (segment (start 197.628 84.36) (end 200.66 84.36) (width 0.25) (layer "F.Cu") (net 8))
 (segment (start 200.406 83.058) (end 200.66 83.312) (width 0.25) (layer "F.Cu") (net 8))
 (segment (start 182.9015 88.138) (end 182.9015 91.694) (width 0.25) (layer "F.Cu") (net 8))
 (segment (start 184.0465 91.694) (end 182.9015 91.694) (width 0.25) (layer "F.Cu") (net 8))
 (segment (start 185.502 90.2385) (end 184.0465 91.694) (width 0.25) (layer "F.Cu") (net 8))
 (segment (start 199.39 83.058) (end 200.406 83.058) (width 0.25) (layer "F.Cu") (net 8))
 (segment (start 200.66 83.312) (end 200.66 84.36) (width 0.25) (layer "F.Cu") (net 8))
 (segment (start 194.564 84.36) (end 197.596 84.36) (width 0.25) (layer "F.Cu") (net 8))
 (segment (start 182.9015 86.8895) (end 182.372 86.36) (width 0.25) (layer "F.Cu") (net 8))
 (segment (start 182.9015 88.138) (end 182.9015 86.8895) (width 0.25) (layer "F.Cu") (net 8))
 (segment (start 186.802 85.994) (end 184.658 88.138) (width 0.25) (layer "F.Cu") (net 8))
 (segment (start 184.658 88.138) (end 182.9015 88.138) (width 0.25) (layer "F.Cu") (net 8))
 (segment (start 197.596 84.36) (end 197.612 84.344) (width 0.25) (layer "F.Cu") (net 8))
 (via (at 199.39 83.058) (size 0.8) (drill 0.4) (layers "F.Cu" "B.Cu") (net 8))
 (via (at 182.372 86.36) (size 0.8) (drill 0.4) (layers "F.Cu" "B.Cu") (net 8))
 (segment (start 182.372 86.36) (end 181.864 85.852) (width 0.25) (layer "B.Cu") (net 8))
 (segment (start 181.864 85.852) (end 181.864 83.82) (width 0.25) (layer "B.Cu") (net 8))
 (segment (start 182.626 83.058) (end 199.39 83.058) (width 0.25) (layer "B.Cu") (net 8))
 (segment (start 181.864 83.82) (end 182.626 83.058) (width 0.25) (layer "B.Cu") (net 8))
 (segment (start 186.6685 81.28) (end 187.452 82.0635) (width 0.25) (layer "F.Cu") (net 1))
 (segment (start 184.642 81.28) (end 184.642 82.8415) (width 0.25) (layer "F.Cu") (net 1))
 (segment (start 184.642 82.8415) (end 182.9015 84.582) (width 0.25) (layer "F.Cu") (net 1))
 (segment (start 186.6685 81.28) (end 184.642 81.28) (width 0.25) (layer "F.Cu") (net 1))
 (segment (start 187.452 82.0635) (end 187.452 84.5135) (width 0.25) (layer "F.Cu") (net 1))
 (segment (start 192.786 71.628) (end 192.786 81.264) (width 1) (layer "F.Cu") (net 7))
 (segment (start 193.294 81.804) (end 192.77 81.28) (width 0.25) (layer "F.Cu") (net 7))
 (segment (start 190.246 83.312) (end 190.246 85.09) (width 0.25) (layer "F.Cu") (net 7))
 (segment (start 189.992 83.058) (end 190.246 83.312) (width 0.25) (layer "F.Cu") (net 7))
 (segment (start 192.786 85.344) (end 193.294 84.836) (width 0.25) (layer "F.Cu") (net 7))
 (segment (start 188.752 83.536) (end 189.23 83.058) (width 0.25) (layer "F.Cu") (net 7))
 (segment (start 188.752 84.5135) (end 188.752 83.536) (width 0.25) (layer "F.Cu") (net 7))
 (segment (start 190.217 69.342) (end 190.5 69.342) (width 0.25) (layer "F.Cu") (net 7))
 (segment (start 190.5 69.342) (end 192.786 71.628) (width 1) (layer "F.Cu") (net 7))
 (segment (start 190.246 85.09) (end 190.5 85.344) (width 0.25) (layer "F.Cu") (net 7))
 (segment (start 190.5 85.344) (end 192.786 85.344) (width 0.25) (layer "F.Cu") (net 7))
 (segment (start 193.294 84.836) (end 193.294 81.804) (width 0.25) (layer "F.Cu") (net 7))
 (segment (start 189.23 83.058) (end 189.992 83.058) (width 0.25) (layer "F.Cu") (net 7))
 (segment (start 192.786 81.264) (end 192.77 81.28) (width 0.25) (layer "F.Cu") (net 7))
 (segment (start 190.77 81.28) (end 190.77 83.3065) (width 0.25) (layer "F.Cu") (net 2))
 (segment (start 188.102 81.9215) (end 188.102 84.634) (width 0.25) (layer "F.Cu") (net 2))
 (segment (start 188.7435 81.28) (end 190.77 81.28) (width 0.25) (layer "F.Cu") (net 2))
 (segment (start 190.77 83.3065) (end 191.77 84.3065) (width 0.25) (layer "F.Cu") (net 2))
 (segment (start 188.7435 81.28) (end 188.102 81.9215) (width 0.25) (layer "F.Cu") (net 2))
 (segment (start 197.612 87.122) (end 197.612 86.344) (width 0.25) (layer "F.Cu") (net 10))
 (segment (start 191.77 89.916) (end 190.5 88.646) (width 0.25) (layer "F.Cu") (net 10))
 (segment (start 187.055959 88.646) (end 186.152 89.549959) (width 0.25) (layer "F.Cu") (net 10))
 (segment (start 186.152 89.549959) (end 186.152 90.2385) (width 0.25) (layer "F.Cu") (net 10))
 (segment (start 196.088 88.646) (end 197.612 87.122) (width 0.25) (layer "F.Cu") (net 10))
 (segment (start 190.5 88.646) (end 187.055959 88.646) (width 0.25) (layer "F.Cu") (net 10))
 (segment (start 197.612 86.344) (end 197.612 91.186) (width 0.25) (layer "F.Cu") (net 10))
 (via (at 191.77 89.916) (size 0.8) (drill 0.4) (layers "F.Cu" "B.Cu") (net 10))
 (via (at 196.088 88.646) (size 0.8) (drill 0.4) (layers "F.Cu" "B.Cu") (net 10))
 (segment (start 193.04 88.646) (end 196.088 88.646) (width 0.25) (layer "B.Cu") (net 10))
 (segment (start 191.77 89.916) (end 193.04 88.646) (width 0.25) (layer "B.Cu") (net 10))
 (segment (start 193.04 90.17) (end 194.564 88.646) (width 0.25) (layer "F.Cu") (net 11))
 (segment (start 194.564 86.36) (end 194.564 91.177) (width 0.25) (layer "F.Cu") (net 11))
 (segment (start 194.564 88.646) (end 194.564 86.36) (width 0.25) (layer "F.Cu") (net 11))
 (segment (start 186.802 92.06) (end 187.706 92.964) (width 0.25) (layer "F.Cu") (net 11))
 (segment (start 186.802 90.2385) (end 186.802 92.06) (width 0.25) (layer "F.Cu") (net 11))
 (segment (start 187.706 92.964) (end 191.516 92.964) (width 0.25) (layer "F.Cu") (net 11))
 (segment (start 193.04 91.44) (end 193.04 90.17) (width 0.25) (layer "F.Cu") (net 11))
 (segment (start 191.516 92.964) (end 193.04 91.44) (width 0.25) (layer "F.Cu") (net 11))
 (segment (start 200.66 88.392) (end 200.66 86.36) (width 0.25) (layer "F.Cu") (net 13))
 (segment (start 199.39 89.662) (end 200.66 88.392) (width 0.25) (layer "F.Cu") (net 13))
 (segment (start 188.102 90.2385) (end 188.102 91.074) (width 0.25) (layer "F.Cu") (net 13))
 (segment (start 188.102 91.074) (end 188.722 91.694) (width 0.25) (layer "F.Cu") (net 13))
 (segment (start 200.66 86.36) (end 200.66 91.177) (width 0.25) (layer "F.Cu") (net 13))
 (via (at 188.722 91.694) (size 0.8) (drill 0.4) (layers "F.Cu" "B.Cu") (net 13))
 (via (at 199.39 89.662) (size 0.8) (drill 0.4) (layers "F.Cu" "B.Cu") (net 13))
 (segment (start 188.722 91.694) (end 197.358 91.694) (width 0.25) (layer "B.Cu") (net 13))
 (segment (start 197.358 91.694) (end 199.39 89.662) (width 0.25) (layer "B.Cu") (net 13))
 (segment (start 168.365 70.88) (end 170.558 73.073) (width 0.25) (layer "F.Cu") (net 5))
 (segment (start 170.558 73.073) (end 170.558 75.678) (width 0.25) (layer "F.Cu") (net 5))
 (segment (start 168.125 71.12) (end 168.365 70.88) (width 0.25) (layer "F.Cu") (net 5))
 (segment (start 185.217 69.342) (end 184.912 69.342) (width 0.25) (layer "F.Cu") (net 20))
 (segment (start 182.626 81.264) (end 182.642 81.28) (width 0.25) (layer "F.Cu") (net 20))
 (segment (start 182.626 71.628) (end 182.626 81.264) (width 1) (layer "F.Cu") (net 20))
 (segment (start 184.912 69.342) (end 182.626 71.628) (width 1) (layer "F.Cu") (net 20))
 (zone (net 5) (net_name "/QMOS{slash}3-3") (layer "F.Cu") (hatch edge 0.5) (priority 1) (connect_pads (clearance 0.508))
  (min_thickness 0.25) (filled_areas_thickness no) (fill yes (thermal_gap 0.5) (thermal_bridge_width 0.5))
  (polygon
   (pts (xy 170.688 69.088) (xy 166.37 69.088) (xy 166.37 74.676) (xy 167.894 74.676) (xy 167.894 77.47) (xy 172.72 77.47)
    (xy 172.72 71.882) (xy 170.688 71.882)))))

